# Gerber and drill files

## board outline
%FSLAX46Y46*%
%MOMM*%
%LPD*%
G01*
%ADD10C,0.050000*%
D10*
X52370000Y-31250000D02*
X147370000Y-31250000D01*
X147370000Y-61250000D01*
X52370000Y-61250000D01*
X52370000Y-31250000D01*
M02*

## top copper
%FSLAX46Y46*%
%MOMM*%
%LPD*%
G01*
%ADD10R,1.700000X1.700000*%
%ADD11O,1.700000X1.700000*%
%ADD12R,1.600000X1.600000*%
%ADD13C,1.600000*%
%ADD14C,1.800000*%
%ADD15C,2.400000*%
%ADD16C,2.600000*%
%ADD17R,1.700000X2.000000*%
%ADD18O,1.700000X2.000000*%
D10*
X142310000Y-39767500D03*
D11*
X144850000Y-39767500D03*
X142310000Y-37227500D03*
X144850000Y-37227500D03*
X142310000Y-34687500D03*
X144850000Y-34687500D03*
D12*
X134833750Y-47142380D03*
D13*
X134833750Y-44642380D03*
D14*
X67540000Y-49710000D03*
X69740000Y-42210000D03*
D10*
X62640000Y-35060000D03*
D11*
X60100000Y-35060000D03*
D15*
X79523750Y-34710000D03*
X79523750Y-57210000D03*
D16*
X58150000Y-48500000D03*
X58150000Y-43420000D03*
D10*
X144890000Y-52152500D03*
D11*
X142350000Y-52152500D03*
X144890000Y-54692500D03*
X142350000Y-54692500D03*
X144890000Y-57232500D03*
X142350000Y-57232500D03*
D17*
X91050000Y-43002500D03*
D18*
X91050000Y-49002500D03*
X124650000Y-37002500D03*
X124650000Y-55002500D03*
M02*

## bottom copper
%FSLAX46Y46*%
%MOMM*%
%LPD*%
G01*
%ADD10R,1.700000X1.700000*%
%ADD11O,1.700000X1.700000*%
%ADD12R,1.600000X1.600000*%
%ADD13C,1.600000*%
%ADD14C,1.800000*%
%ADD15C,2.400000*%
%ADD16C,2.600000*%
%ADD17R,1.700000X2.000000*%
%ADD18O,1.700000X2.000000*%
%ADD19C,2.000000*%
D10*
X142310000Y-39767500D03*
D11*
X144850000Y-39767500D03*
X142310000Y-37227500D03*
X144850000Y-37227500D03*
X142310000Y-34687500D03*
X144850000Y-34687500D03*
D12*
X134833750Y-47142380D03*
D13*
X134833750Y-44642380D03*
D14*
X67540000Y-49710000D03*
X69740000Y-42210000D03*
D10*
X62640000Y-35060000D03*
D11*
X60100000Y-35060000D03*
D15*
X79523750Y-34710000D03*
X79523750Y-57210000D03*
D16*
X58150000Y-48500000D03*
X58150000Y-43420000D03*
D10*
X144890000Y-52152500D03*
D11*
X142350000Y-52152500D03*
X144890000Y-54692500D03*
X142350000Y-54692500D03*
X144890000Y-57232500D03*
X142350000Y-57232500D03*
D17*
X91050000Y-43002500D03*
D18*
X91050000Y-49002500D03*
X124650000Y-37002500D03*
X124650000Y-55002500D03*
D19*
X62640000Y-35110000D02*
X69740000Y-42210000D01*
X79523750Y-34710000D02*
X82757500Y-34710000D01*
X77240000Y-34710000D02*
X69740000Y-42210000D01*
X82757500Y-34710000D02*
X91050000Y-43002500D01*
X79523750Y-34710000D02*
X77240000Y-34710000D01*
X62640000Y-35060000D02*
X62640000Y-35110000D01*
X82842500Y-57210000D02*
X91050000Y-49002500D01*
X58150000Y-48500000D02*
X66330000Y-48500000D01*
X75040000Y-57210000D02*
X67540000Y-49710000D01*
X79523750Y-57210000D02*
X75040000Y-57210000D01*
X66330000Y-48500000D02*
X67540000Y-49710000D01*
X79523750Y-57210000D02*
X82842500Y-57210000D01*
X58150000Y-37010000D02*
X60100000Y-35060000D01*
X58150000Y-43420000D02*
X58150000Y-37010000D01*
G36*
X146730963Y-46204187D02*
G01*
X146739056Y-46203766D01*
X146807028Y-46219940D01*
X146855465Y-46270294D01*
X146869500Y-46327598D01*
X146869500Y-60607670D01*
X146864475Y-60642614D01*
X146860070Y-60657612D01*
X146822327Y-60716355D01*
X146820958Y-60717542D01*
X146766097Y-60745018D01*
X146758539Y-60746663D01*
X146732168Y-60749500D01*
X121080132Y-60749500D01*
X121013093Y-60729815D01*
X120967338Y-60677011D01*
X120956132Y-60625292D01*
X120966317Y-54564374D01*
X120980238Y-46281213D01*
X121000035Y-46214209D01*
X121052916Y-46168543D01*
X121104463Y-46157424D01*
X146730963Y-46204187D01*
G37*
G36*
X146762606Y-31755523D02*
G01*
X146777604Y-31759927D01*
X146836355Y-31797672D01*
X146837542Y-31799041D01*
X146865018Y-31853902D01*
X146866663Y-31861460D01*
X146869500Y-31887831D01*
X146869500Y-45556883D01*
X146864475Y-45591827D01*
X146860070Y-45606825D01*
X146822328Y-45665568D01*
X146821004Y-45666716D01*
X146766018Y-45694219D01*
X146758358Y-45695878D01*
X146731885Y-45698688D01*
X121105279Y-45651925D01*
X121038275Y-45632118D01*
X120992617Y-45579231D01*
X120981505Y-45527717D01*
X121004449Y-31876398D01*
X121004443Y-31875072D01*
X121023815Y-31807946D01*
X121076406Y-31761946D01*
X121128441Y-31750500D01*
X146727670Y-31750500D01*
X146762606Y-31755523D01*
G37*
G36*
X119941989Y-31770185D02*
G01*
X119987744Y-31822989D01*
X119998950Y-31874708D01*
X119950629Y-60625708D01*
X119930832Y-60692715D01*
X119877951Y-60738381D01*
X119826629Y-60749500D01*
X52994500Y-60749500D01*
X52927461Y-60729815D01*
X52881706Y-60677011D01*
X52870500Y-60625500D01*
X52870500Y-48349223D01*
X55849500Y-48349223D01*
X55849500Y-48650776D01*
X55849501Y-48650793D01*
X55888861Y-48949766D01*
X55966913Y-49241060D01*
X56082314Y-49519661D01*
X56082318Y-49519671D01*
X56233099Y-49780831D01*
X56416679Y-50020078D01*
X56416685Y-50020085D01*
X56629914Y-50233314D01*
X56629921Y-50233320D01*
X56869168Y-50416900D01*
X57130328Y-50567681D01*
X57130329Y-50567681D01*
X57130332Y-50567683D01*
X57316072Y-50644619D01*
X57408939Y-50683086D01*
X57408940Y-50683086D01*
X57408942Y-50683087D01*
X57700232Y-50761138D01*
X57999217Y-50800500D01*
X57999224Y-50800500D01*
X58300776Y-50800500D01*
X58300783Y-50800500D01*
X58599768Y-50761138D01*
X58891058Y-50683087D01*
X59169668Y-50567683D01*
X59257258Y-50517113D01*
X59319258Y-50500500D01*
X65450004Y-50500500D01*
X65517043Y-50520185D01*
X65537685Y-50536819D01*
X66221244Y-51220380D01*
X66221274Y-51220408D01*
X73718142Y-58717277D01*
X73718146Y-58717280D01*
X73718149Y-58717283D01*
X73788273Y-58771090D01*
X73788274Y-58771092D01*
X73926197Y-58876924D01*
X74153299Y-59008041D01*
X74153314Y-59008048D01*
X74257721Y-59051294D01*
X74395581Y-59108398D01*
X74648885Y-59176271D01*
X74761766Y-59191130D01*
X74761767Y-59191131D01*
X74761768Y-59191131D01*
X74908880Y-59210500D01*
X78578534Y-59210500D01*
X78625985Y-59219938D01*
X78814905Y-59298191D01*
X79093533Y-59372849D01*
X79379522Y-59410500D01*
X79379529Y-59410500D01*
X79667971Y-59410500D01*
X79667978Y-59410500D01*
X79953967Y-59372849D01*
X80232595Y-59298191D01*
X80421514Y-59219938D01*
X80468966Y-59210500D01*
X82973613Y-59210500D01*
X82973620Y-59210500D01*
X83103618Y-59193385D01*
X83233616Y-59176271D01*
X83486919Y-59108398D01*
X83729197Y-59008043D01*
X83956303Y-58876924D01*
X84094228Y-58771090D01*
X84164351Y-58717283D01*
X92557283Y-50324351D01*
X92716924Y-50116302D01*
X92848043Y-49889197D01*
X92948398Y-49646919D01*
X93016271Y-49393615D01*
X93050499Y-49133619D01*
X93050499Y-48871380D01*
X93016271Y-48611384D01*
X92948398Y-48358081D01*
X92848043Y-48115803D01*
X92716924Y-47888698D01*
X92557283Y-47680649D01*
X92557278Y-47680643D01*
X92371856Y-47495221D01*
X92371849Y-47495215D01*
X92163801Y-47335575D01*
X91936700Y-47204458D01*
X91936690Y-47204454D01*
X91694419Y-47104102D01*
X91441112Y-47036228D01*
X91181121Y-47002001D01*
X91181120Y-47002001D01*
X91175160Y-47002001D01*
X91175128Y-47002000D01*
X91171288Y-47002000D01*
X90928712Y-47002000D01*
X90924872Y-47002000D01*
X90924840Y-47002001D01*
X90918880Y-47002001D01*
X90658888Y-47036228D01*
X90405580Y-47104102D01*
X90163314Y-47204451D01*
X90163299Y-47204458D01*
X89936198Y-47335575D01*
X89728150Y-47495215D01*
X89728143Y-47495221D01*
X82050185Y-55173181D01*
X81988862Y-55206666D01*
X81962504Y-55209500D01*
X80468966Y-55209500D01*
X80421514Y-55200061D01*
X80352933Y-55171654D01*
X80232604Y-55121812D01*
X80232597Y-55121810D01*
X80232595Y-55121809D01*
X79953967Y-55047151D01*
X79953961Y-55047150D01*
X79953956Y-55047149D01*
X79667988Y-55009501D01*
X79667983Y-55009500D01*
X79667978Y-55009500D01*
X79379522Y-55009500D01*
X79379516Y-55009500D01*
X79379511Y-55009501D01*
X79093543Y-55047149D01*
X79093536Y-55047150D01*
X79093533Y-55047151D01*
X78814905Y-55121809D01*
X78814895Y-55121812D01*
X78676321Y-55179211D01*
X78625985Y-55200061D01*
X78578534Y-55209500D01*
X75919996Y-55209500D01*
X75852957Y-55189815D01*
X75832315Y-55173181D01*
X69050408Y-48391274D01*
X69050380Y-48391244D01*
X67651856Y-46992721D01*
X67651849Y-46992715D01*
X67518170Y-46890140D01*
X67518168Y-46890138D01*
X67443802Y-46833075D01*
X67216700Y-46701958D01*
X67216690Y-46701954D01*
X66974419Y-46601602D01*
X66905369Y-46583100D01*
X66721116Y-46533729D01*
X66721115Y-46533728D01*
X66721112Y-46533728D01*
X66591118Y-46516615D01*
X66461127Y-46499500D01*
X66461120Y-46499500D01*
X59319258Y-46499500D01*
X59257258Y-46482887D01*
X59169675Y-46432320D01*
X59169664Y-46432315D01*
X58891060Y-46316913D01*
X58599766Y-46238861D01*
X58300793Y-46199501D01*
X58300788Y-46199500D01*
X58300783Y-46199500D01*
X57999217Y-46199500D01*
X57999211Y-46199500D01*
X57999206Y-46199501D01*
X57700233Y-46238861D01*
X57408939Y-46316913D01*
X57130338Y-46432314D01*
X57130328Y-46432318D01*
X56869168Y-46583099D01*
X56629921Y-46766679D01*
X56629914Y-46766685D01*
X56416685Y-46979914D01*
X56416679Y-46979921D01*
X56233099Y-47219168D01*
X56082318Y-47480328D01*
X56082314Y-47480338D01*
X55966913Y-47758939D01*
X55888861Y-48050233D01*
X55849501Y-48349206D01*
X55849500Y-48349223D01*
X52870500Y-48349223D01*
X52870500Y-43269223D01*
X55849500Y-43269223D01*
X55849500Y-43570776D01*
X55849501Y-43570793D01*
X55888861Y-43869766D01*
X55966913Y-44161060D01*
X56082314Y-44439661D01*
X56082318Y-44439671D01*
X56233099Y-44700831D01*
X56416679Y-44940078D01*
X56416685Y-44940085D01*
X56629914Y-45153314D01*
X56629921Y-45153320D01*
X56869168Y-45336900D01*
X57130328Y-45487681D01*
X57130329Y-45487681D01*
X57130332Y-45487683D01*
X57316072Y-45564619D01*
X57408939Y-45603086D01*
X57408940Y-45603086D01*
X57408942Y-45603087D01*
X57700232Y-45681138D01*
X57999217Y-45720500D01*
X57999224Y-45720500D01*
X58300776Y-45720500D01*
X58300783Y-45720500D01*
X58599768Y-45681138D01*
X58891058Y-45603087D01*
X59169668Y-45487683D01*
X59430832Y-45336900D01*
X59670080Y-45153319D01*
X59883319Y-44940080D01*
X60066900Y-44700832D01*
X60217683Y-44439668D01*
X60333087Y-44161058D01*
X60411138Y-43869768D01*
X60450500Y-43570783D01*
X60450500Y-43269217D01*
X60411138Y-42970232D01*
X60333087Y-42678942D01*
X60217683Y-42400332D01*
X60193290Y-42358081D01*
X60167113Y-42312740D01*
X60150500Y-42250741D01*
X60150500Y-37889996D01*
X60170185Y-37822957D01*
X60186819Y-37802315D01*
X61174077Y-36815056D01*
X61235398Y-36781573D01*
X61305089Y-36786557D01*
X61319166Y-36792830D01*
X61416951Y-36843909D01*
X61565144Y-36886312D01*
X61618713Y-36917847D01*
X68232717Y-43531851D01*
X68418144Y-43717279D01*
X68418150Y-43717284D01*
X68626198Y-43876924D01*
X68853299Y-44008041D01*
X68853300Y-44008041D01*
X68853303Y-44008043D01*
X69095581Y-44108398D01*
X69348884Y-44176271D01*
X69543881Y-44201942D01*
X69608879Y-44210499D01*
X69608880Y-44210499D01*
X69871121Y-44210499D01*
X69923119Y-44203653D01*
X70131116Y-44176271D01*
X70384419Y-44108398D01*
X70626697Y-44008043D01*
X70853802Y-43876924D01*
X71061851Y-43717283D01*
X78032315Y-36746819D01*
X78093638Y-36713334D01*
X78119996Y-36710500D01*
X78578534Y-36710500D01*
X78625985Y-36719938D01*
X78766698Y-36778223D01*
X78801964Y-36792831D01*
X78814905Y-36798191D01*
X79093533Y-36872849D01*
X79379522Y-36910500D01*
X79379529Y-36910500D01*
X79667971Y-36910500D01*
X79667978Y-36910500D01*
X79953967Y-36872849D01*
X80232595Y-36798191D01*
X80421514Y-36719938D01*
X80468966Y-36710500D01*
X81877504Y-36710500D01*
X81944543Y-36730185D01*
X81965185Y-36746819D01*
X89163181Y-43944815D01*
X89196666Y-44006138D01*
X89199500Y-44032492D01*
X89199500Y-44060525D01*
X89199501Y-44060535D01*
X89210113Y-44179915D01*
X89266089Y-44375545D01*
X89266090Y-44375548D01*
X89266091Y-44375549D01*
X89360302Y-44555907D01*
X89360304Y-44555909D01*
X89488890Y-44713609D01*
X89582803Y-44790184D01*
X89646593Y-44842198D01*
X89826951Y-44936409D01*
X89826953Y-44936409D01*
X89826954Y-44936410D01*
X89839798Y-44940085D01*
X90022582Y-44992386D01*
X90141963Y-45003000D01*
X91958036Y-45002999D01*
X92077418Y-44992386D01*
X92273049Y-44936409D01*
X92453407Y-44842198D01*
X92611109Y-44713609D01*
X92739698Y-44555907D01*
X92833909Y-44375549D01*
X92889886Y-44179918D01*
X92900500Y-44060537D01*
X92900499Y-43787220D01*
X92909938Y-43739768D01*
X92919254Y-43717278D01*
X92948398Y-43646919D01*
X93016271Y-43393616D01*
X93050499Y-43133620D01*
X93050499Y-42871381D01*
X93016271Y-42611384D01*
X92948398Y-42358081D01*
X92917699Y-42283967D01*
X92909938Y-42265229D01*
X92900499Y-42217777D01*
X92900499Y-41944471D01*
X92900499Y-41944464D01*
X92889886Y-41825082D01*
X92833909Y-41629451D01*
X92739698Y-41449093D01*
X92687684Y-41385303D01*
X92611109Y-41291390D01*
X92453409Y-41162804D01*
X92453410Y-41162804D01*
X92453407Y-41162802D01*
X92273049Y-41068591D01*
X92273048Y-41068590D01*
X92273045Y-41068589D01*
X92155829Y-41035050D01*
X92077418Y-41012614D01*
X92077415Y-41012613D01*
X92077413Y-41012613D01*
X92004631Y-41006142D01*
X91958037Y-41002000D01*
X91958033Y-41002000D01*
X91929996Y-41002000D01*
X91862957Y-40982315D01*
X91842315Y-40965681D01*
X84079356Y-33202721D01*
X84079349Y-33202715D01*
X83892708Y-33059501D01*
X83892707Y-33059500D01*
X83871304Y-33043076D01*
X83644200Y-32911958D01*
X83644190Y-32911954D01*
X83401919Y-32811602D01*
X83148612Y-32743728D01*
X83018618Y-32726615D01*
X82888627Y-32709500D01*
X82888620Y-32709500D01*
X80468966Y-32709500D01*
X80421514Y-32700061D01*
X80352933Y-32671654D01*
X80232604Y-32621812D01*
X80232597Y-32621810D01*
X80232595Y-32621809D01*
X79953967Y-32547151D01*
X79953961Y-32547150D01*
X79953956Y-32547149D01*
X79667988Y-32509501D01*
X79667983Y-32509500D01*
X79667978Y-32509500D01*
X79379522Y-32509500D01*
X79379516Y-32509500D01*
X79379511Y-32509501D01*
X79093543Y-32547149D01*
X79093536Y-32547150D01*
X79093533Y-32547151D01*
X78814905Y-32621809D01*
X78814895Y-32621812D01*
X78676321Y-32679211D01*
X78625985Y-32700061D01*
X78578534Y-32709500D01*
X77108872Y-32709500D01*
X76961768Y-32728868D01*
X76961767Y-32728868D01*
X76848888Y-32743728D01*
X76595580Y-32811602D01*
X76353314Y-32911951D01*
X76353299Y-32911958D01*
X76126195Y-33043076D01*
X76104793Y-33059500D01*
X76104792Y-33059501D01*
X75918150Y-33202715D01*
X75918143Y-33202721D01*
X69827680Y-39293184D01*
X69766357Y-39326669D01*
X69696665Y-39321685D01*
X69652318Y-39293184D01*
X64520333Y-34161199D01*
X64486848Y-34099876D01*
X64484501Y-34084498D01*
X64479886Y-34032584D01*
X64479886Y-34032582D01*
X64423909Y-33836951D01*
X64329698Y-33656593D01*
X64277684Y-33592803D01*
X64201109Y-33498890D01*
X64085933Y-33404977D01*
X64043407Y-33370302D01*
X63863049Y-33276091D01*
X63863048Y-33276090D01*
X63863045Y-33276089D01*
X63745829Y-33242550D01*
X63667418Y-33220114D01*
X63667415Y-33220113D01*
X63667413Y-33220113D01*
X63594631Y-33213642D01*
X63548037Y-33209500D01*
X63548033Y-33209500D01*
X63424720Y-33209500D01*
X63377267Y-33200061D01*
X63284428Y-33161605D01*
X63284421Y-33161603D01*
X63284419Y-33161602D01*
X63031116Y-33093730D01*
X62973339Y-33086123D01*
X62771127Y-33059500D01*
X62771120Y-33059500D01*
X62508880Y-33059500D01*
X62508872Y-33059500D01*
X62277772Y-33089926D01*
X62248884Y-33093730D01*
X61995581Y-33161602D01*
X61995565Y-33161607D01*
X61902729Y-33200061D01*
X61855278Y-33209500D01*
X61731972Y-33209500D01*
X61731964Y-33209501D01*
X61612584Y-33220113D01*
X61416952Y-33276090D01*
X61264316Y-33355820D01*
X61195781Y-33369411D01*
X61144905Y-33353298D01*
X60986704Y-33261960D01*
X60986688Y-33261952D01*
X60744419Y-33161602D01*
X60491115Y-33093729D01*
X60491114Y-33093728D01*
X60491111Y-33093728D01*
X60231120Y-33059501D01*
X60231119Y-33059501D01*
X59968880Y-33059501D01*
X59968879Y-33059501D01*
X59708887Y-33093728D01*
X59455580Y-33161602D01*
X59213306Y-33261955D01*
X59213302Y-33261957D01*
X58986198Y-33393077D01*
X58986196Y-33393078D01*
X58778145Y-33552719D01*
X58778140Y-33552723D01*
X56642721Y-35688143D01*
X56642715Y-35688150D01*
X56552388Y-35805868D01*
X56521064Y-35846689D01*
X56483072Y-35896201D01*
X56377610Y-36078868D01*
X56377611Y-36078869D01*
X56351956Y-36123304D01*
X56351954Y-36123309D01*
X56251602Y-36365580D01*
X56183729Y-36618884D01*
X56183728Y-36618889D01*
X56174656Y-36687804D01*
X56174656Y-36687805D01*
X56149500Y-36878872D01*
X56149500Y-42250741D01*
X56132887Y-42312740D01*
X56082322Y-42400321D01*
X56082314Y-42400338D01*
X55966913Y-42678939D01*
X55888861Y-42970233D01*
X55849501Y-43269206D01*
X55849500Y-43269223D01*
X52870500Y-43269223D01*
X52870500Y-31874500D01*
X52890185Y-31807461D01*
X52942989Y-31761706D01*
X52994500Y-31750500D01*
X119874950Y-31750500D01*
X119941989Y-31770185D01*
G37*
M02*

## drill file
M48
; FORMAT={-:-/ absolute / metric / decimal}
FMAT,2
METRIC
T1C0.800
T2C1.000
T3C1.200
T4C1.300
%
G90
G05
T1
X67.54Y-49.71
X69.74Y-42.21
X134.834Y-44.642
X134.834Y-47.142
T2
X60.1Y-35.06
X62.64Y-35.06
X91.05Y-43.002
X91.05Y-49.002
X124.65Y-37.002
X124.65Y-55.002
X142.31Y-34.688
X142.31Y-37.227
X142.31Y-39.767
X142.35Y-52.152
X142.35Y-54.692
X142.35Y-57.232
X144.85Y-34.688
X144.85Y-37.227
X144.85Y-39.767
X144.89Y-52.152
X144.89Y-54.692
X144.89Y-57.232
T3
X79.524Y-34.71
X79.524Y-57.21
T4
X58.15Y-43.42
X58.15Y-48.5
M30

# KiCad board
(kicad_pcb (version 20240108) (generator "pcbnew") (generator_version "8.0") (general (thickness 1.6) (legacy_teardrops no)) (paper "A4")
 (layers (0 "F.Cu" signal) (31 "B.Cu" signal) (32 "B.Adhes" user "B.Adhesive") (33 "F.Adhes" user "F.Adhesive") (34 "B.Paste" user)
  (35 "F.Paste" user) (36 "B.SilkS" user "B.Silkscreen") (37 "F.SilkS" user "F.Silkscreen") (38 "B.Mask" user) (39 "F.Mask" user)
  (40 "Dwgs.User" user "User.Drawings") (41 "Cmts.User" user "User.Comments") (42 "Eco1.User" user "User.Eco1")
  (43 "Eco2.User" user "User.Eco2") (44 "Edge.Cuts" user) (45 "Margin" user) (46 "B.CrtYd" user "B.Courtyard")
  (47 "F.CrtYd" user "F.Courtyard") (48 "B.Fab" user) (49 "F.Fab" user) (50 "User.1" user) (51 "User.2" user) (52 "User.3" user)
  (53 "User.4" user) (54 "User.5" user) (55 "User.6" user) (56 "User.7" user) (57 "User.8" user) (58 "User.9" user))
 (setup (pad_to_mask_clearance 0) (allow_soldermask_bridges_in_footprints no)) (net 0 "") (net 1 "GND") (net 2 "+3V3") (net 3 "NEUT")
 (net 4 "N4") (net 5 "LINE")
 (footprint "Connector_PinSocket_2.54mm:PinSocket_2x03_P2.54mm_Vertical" (layer "F.Cu") (at 142.31 39.7675 180)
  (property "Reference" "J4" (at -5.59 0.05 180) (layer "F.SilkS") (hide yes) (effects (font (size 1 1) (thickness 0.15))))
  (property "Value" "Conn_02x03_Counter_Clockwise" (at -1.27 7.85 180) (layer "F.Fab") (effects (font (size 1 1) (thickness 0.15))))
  (pad "1" thru_hole rect (at 0 0 180) (size 1.7 1.7) (drill 1) (layers "*.Cu" "*.Mask") (remove_unused_layers no) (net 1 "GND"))
  (pad "2" thru_hole oval (at -2.54 0 180) (size 1.7 1.7) (drill 1) (layers "*.Cu" "*.Mask") (remove_unused_layers no) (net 1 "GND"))
  (pad "3" thru_hole oval (at 0 2.54 180) (size 1.7 1.7) (drill 1) (layers "*.Cu" "*.Mask") (remove_unused_layers no) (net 1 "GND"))
  (pad "4" thru_hole oval (at -2.54 2.54 180) (size 1.7 1.7) (drill 1) (layers "*.Cu" "*.Mask") (remove_unused_layers no) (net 1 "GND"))
  (pad "5" thru_hole oval (at 0 5.08 180) (size 1.7 1.7) (drill 1) (layers "*.Cu" "*.Mask") (remove_unused_layers no) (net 1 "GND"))
  (pad "6" thru_hole oval (at -2.54 5.08 180) (size 1.7 1.7) (drill 1) (layers "*.Cu" "*.Mask") (remove_unused_layers no) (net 1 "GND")))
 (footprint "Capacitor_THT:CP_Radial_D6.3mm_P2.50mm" (layer "F.Cu") (at 134.83375 47.14238 90)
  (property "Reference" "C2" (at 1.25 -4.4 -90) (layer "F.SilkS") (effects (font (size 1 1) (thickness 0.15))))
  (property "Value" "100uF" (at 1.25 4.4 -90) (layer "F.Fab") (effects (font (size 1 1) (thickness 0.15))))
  (pad "1" thru_hole rect (at 0 0 90) (size 1.6 1.6) (drill 0.8) (layers "*.Cu" "*.Mask") (remove_unused_layers no) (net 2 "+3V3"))
  (pad "2" thru_hole circle (at 2.5 0 90) (size 1.6 1.6) (drill 0.8) (layers "*.Cu" "*.Mask") (remove_unused_layers no) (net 1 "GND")))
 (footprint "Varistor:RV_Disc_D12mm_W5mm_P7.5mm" (layer "F.Cu") (at 67.54 49.71 90)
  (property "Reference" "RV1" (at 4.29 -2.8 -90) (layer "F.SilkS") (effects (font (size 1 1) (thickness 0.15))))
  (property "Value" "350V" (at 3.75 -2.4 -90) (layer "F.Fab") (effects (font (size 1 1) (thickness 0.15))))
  (pad "1" thru_hole circle (at 0 0 90) (size 1.8 1.8) (drill 0.8) (layers "*.Cu" "*.Mask") (remove_unused_layers no) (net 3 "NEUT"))
  (pad "2" thru_hole circle (at 7.5 2.2 90) (size 1.8 1.8) (drill 0.8) (layers "*.Cu" "*.Mask") (remove_unused_layers no) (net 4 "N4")))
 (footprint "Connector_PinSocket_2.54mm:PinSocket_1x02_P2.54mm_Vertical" (layer "F.Cu") (at 62.64 35.06 -90)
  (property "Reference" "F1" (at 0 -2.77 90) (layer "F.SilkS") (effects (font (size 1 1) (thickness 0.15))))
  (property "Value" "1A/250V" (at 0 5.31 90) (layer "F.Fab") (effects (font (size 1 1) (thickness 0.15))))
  (pad "1" thru_hole rect (at 0 0 270) (size 1.7 1.7) (drill 1) (layers "*.Cu" "*.Mask") (remove_unused_layers no) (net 4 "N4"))
  (pad "2" thru_hole oval (at 0 2.54 270) (size 1.7 1.7) (drill 1) (layers "*.Cu" "*.Mask") (remove_unused_layers no) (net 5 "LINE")))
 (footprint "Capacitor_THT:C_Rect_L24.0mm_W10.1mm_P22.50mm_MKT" (layer "F.Cu") (at 79.52375 34.71 -90)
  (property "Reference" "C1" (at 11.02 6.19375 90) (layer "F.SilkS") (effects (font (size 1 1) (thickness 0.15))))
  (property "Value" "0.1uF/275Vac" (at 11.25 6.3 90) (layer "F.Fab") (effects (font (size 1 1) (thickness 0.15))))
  (pad "1" thru_hole circle (at 0 0 270) (size 2.4 2.4) (drill 1.2) (layers "*.Cu" "*.Mask") (remove_unused_layers no) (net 4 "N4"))
  (pad "2" thru_hole circle (at 22.5 0 270) (size 2.4 2.4) (drill 1.2) (layers "*.Cu" "*.Mask") (remove_unused_layers no) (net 3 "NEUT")))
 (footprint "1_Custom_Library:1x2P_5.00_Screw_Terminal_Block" (layer "F.Cu") (at 58.3 46.75 180)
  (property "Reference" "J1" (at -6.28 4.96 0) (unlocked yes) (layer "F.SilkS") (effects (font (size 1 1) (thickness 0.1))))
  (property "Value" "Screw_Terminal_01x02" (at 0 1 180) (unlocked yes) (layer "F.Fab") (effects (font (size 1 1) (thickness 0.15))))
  (pad "1" thru_hole circle (at 0.15 -1.75 180) (size 2.6 2.6) (drill 1.3) (layers "*.Cu" "*.Mask") (remove_unused_layers no) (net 3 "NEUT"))
  (pad "2" thru_hole circle (at 0.15 3.33 180) (size 2.6 2.6) (drill 1.3) (layers "*.Cu" "*.Mask") (remove_unused_layers no) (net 5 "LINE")))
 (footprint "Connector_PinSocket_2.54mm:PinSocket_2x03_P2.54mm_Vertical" (layer "F.Cu") (at 144.89 52.1525)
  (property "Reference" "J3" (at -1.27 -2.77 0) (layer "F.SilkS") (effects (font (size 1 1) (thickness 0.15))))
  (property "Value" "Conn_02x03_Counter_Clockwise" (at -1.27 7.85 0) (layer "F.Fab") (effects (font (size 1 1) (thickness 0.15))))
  (pad "1" thru_hole rect (at 0 0) (size 1.7 1.7) (drill 1) (layers "*.Cu" "*.Mask") (remove_unused_layers no) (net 2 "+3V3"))
  (pad "2" thru_hole oval (at -2.54 0) (size 1.7 1.7) (drill 1) (layers "*.Cu" "*.Mask") (remove_unused_layers no) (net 2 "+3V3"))
  (pad "3" thru_hole oval (at 0 2.54) (size 1.7 1.7) (drill 1) (layers "*.Cu" "*.Mask") (remove_unused_layers no) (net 2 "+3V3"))
  (pad "4" thru_hole oval (at -2.54 2.54) (size 1.7 1.7) (drill 1) (layers "*.Cu" "*.Mask") (remove_unused_layers no) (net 2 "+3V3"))
  (pad "5" thru_hole oval (at 0 5.08) (size 1.7 1.7) (drill 1) (layers "*.Cu" "*.Mask") (remove_unused_layers no) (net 2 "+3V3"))
  (pad "6" thru_hole oval (at -2.54 5.08) (size 1.7 1.7) (drill 1) (layers "*.Cu" "*.Mask") (remove_unused_layers no) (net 2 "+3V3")))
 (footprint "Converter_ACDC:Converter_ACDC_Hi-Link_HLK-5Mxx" (layer "F.Cu") (at 91.05 43.0025)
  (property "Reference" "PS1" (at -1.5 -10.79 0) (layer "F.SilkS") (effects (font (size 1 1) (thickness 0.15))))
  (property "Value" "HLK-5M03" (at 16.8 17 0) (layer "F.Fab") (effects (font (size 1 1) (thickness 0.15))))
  (pad "1" thru_hole rect (at 0 0) (size 1.7 2) (drill 1) (layers "*.Cu" "*.Mask") (remove_unused_layers no) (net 4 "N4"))
  (pad "2" thru_hole oval (at 0 6) (size 1.7 2) (drill 1) (layers "*.Cu" "*.Mask") (remove_unused_layers no) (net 3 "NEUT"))
  (pad "3" thru_hole oval (at 33.6 -6) (size 1.7 2) (drill 1) (layers "*.Cu" "*.Mask") (remove_unused_layers no) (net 1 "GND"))
  (pad "4" thru_hole oval (at 33.6 12) (size 1.7 2) (drill 1) (layers "*.Cu" "*.Mask") (remove_unused_layers no) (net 2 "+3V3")))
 (gr_rect (start 52.37 31.25) (end 147.37 61.25) (stroke (width 0.05) (type default)) (fill none) (layer "Edge.Cuts"))
 (segment (start 62.64 35.11) (end 69.74 42.21) (width 2) (layer "B.Cu") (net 4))
 (segment (start 79.52375 34.71) (end 82.7575 34.71) (width 2) (layer "B.Cu") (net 4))
 (segment (start 77.24 34.71) (end 69.74 42.21) (width 2) (layer "B.Cu") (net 4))
 (segment (start 82.7575 34.71) (end 91.05 43.0025) (width 2) (layer "B.Cu") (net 4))
 (segment (start 79.52375 34.71) (end 77.24 34.71) (width 2) (layer "B.Cu") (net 4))
 (segment (start 62.64 35.06) (end 62.64 35.11) (width 2) (layer "B.Cu") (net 4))
 (segment (start 82.8425 57.21) (end 91.05 49.0025) (width 2) (layer "B.Cu") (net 3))
 (segment (start 58.15 48.5) (end 66.33 48.5) (width 2) (layer "B.Cu") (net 3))
 (segment (start 75.04 57.21) (end 67.54 49.71) (width 2) (layer "B.Cu") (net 3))
 (segment (start 79.52375 57.21) (end 75.04 57.21) (width 2) (layer "B.Cu") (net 3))
 (segment (start 66.33 48.5) (end 67.54 49.71) (width 2) (layer "B.Cu") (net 3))
 (segment (start 79.52375 57.21) (end 82.8425 57.21) (width 2) (layer "B.Cu") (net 3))
 (segment (start 58.15 37.01) (end 60.1 35.06) (width 2) (layer "B.Cu") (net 5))
 (segment (start 58.15 43.42) (end 58.15 37.01) (width 2) (layer "B.Cu") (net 5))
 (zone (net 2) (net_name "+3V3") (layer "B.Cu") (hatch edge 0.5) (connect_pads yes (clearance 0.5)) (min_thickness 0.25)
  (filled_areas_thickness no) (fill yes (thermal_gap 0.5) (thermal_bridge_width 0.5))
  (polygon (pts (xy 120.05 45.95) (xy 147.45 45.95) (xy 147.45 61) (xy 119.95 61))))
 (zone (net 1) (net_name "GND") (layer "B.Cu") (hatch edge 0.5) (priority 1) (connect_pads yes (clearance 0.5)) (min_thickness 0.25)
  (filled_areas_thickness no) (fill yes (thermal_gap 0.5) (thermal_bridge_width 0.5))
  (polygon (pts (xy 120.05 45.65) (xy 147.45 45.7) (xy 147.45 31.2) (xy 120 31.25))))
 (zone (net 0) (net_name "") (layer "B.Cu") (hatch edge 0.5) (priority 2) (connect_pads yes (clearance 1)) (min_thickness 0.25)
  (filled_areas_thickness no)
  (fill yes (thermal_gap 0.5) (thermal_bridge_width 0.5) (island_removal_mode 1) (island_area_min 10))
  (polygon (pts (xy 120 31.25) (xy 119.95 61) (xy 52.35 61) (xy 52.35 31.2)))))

